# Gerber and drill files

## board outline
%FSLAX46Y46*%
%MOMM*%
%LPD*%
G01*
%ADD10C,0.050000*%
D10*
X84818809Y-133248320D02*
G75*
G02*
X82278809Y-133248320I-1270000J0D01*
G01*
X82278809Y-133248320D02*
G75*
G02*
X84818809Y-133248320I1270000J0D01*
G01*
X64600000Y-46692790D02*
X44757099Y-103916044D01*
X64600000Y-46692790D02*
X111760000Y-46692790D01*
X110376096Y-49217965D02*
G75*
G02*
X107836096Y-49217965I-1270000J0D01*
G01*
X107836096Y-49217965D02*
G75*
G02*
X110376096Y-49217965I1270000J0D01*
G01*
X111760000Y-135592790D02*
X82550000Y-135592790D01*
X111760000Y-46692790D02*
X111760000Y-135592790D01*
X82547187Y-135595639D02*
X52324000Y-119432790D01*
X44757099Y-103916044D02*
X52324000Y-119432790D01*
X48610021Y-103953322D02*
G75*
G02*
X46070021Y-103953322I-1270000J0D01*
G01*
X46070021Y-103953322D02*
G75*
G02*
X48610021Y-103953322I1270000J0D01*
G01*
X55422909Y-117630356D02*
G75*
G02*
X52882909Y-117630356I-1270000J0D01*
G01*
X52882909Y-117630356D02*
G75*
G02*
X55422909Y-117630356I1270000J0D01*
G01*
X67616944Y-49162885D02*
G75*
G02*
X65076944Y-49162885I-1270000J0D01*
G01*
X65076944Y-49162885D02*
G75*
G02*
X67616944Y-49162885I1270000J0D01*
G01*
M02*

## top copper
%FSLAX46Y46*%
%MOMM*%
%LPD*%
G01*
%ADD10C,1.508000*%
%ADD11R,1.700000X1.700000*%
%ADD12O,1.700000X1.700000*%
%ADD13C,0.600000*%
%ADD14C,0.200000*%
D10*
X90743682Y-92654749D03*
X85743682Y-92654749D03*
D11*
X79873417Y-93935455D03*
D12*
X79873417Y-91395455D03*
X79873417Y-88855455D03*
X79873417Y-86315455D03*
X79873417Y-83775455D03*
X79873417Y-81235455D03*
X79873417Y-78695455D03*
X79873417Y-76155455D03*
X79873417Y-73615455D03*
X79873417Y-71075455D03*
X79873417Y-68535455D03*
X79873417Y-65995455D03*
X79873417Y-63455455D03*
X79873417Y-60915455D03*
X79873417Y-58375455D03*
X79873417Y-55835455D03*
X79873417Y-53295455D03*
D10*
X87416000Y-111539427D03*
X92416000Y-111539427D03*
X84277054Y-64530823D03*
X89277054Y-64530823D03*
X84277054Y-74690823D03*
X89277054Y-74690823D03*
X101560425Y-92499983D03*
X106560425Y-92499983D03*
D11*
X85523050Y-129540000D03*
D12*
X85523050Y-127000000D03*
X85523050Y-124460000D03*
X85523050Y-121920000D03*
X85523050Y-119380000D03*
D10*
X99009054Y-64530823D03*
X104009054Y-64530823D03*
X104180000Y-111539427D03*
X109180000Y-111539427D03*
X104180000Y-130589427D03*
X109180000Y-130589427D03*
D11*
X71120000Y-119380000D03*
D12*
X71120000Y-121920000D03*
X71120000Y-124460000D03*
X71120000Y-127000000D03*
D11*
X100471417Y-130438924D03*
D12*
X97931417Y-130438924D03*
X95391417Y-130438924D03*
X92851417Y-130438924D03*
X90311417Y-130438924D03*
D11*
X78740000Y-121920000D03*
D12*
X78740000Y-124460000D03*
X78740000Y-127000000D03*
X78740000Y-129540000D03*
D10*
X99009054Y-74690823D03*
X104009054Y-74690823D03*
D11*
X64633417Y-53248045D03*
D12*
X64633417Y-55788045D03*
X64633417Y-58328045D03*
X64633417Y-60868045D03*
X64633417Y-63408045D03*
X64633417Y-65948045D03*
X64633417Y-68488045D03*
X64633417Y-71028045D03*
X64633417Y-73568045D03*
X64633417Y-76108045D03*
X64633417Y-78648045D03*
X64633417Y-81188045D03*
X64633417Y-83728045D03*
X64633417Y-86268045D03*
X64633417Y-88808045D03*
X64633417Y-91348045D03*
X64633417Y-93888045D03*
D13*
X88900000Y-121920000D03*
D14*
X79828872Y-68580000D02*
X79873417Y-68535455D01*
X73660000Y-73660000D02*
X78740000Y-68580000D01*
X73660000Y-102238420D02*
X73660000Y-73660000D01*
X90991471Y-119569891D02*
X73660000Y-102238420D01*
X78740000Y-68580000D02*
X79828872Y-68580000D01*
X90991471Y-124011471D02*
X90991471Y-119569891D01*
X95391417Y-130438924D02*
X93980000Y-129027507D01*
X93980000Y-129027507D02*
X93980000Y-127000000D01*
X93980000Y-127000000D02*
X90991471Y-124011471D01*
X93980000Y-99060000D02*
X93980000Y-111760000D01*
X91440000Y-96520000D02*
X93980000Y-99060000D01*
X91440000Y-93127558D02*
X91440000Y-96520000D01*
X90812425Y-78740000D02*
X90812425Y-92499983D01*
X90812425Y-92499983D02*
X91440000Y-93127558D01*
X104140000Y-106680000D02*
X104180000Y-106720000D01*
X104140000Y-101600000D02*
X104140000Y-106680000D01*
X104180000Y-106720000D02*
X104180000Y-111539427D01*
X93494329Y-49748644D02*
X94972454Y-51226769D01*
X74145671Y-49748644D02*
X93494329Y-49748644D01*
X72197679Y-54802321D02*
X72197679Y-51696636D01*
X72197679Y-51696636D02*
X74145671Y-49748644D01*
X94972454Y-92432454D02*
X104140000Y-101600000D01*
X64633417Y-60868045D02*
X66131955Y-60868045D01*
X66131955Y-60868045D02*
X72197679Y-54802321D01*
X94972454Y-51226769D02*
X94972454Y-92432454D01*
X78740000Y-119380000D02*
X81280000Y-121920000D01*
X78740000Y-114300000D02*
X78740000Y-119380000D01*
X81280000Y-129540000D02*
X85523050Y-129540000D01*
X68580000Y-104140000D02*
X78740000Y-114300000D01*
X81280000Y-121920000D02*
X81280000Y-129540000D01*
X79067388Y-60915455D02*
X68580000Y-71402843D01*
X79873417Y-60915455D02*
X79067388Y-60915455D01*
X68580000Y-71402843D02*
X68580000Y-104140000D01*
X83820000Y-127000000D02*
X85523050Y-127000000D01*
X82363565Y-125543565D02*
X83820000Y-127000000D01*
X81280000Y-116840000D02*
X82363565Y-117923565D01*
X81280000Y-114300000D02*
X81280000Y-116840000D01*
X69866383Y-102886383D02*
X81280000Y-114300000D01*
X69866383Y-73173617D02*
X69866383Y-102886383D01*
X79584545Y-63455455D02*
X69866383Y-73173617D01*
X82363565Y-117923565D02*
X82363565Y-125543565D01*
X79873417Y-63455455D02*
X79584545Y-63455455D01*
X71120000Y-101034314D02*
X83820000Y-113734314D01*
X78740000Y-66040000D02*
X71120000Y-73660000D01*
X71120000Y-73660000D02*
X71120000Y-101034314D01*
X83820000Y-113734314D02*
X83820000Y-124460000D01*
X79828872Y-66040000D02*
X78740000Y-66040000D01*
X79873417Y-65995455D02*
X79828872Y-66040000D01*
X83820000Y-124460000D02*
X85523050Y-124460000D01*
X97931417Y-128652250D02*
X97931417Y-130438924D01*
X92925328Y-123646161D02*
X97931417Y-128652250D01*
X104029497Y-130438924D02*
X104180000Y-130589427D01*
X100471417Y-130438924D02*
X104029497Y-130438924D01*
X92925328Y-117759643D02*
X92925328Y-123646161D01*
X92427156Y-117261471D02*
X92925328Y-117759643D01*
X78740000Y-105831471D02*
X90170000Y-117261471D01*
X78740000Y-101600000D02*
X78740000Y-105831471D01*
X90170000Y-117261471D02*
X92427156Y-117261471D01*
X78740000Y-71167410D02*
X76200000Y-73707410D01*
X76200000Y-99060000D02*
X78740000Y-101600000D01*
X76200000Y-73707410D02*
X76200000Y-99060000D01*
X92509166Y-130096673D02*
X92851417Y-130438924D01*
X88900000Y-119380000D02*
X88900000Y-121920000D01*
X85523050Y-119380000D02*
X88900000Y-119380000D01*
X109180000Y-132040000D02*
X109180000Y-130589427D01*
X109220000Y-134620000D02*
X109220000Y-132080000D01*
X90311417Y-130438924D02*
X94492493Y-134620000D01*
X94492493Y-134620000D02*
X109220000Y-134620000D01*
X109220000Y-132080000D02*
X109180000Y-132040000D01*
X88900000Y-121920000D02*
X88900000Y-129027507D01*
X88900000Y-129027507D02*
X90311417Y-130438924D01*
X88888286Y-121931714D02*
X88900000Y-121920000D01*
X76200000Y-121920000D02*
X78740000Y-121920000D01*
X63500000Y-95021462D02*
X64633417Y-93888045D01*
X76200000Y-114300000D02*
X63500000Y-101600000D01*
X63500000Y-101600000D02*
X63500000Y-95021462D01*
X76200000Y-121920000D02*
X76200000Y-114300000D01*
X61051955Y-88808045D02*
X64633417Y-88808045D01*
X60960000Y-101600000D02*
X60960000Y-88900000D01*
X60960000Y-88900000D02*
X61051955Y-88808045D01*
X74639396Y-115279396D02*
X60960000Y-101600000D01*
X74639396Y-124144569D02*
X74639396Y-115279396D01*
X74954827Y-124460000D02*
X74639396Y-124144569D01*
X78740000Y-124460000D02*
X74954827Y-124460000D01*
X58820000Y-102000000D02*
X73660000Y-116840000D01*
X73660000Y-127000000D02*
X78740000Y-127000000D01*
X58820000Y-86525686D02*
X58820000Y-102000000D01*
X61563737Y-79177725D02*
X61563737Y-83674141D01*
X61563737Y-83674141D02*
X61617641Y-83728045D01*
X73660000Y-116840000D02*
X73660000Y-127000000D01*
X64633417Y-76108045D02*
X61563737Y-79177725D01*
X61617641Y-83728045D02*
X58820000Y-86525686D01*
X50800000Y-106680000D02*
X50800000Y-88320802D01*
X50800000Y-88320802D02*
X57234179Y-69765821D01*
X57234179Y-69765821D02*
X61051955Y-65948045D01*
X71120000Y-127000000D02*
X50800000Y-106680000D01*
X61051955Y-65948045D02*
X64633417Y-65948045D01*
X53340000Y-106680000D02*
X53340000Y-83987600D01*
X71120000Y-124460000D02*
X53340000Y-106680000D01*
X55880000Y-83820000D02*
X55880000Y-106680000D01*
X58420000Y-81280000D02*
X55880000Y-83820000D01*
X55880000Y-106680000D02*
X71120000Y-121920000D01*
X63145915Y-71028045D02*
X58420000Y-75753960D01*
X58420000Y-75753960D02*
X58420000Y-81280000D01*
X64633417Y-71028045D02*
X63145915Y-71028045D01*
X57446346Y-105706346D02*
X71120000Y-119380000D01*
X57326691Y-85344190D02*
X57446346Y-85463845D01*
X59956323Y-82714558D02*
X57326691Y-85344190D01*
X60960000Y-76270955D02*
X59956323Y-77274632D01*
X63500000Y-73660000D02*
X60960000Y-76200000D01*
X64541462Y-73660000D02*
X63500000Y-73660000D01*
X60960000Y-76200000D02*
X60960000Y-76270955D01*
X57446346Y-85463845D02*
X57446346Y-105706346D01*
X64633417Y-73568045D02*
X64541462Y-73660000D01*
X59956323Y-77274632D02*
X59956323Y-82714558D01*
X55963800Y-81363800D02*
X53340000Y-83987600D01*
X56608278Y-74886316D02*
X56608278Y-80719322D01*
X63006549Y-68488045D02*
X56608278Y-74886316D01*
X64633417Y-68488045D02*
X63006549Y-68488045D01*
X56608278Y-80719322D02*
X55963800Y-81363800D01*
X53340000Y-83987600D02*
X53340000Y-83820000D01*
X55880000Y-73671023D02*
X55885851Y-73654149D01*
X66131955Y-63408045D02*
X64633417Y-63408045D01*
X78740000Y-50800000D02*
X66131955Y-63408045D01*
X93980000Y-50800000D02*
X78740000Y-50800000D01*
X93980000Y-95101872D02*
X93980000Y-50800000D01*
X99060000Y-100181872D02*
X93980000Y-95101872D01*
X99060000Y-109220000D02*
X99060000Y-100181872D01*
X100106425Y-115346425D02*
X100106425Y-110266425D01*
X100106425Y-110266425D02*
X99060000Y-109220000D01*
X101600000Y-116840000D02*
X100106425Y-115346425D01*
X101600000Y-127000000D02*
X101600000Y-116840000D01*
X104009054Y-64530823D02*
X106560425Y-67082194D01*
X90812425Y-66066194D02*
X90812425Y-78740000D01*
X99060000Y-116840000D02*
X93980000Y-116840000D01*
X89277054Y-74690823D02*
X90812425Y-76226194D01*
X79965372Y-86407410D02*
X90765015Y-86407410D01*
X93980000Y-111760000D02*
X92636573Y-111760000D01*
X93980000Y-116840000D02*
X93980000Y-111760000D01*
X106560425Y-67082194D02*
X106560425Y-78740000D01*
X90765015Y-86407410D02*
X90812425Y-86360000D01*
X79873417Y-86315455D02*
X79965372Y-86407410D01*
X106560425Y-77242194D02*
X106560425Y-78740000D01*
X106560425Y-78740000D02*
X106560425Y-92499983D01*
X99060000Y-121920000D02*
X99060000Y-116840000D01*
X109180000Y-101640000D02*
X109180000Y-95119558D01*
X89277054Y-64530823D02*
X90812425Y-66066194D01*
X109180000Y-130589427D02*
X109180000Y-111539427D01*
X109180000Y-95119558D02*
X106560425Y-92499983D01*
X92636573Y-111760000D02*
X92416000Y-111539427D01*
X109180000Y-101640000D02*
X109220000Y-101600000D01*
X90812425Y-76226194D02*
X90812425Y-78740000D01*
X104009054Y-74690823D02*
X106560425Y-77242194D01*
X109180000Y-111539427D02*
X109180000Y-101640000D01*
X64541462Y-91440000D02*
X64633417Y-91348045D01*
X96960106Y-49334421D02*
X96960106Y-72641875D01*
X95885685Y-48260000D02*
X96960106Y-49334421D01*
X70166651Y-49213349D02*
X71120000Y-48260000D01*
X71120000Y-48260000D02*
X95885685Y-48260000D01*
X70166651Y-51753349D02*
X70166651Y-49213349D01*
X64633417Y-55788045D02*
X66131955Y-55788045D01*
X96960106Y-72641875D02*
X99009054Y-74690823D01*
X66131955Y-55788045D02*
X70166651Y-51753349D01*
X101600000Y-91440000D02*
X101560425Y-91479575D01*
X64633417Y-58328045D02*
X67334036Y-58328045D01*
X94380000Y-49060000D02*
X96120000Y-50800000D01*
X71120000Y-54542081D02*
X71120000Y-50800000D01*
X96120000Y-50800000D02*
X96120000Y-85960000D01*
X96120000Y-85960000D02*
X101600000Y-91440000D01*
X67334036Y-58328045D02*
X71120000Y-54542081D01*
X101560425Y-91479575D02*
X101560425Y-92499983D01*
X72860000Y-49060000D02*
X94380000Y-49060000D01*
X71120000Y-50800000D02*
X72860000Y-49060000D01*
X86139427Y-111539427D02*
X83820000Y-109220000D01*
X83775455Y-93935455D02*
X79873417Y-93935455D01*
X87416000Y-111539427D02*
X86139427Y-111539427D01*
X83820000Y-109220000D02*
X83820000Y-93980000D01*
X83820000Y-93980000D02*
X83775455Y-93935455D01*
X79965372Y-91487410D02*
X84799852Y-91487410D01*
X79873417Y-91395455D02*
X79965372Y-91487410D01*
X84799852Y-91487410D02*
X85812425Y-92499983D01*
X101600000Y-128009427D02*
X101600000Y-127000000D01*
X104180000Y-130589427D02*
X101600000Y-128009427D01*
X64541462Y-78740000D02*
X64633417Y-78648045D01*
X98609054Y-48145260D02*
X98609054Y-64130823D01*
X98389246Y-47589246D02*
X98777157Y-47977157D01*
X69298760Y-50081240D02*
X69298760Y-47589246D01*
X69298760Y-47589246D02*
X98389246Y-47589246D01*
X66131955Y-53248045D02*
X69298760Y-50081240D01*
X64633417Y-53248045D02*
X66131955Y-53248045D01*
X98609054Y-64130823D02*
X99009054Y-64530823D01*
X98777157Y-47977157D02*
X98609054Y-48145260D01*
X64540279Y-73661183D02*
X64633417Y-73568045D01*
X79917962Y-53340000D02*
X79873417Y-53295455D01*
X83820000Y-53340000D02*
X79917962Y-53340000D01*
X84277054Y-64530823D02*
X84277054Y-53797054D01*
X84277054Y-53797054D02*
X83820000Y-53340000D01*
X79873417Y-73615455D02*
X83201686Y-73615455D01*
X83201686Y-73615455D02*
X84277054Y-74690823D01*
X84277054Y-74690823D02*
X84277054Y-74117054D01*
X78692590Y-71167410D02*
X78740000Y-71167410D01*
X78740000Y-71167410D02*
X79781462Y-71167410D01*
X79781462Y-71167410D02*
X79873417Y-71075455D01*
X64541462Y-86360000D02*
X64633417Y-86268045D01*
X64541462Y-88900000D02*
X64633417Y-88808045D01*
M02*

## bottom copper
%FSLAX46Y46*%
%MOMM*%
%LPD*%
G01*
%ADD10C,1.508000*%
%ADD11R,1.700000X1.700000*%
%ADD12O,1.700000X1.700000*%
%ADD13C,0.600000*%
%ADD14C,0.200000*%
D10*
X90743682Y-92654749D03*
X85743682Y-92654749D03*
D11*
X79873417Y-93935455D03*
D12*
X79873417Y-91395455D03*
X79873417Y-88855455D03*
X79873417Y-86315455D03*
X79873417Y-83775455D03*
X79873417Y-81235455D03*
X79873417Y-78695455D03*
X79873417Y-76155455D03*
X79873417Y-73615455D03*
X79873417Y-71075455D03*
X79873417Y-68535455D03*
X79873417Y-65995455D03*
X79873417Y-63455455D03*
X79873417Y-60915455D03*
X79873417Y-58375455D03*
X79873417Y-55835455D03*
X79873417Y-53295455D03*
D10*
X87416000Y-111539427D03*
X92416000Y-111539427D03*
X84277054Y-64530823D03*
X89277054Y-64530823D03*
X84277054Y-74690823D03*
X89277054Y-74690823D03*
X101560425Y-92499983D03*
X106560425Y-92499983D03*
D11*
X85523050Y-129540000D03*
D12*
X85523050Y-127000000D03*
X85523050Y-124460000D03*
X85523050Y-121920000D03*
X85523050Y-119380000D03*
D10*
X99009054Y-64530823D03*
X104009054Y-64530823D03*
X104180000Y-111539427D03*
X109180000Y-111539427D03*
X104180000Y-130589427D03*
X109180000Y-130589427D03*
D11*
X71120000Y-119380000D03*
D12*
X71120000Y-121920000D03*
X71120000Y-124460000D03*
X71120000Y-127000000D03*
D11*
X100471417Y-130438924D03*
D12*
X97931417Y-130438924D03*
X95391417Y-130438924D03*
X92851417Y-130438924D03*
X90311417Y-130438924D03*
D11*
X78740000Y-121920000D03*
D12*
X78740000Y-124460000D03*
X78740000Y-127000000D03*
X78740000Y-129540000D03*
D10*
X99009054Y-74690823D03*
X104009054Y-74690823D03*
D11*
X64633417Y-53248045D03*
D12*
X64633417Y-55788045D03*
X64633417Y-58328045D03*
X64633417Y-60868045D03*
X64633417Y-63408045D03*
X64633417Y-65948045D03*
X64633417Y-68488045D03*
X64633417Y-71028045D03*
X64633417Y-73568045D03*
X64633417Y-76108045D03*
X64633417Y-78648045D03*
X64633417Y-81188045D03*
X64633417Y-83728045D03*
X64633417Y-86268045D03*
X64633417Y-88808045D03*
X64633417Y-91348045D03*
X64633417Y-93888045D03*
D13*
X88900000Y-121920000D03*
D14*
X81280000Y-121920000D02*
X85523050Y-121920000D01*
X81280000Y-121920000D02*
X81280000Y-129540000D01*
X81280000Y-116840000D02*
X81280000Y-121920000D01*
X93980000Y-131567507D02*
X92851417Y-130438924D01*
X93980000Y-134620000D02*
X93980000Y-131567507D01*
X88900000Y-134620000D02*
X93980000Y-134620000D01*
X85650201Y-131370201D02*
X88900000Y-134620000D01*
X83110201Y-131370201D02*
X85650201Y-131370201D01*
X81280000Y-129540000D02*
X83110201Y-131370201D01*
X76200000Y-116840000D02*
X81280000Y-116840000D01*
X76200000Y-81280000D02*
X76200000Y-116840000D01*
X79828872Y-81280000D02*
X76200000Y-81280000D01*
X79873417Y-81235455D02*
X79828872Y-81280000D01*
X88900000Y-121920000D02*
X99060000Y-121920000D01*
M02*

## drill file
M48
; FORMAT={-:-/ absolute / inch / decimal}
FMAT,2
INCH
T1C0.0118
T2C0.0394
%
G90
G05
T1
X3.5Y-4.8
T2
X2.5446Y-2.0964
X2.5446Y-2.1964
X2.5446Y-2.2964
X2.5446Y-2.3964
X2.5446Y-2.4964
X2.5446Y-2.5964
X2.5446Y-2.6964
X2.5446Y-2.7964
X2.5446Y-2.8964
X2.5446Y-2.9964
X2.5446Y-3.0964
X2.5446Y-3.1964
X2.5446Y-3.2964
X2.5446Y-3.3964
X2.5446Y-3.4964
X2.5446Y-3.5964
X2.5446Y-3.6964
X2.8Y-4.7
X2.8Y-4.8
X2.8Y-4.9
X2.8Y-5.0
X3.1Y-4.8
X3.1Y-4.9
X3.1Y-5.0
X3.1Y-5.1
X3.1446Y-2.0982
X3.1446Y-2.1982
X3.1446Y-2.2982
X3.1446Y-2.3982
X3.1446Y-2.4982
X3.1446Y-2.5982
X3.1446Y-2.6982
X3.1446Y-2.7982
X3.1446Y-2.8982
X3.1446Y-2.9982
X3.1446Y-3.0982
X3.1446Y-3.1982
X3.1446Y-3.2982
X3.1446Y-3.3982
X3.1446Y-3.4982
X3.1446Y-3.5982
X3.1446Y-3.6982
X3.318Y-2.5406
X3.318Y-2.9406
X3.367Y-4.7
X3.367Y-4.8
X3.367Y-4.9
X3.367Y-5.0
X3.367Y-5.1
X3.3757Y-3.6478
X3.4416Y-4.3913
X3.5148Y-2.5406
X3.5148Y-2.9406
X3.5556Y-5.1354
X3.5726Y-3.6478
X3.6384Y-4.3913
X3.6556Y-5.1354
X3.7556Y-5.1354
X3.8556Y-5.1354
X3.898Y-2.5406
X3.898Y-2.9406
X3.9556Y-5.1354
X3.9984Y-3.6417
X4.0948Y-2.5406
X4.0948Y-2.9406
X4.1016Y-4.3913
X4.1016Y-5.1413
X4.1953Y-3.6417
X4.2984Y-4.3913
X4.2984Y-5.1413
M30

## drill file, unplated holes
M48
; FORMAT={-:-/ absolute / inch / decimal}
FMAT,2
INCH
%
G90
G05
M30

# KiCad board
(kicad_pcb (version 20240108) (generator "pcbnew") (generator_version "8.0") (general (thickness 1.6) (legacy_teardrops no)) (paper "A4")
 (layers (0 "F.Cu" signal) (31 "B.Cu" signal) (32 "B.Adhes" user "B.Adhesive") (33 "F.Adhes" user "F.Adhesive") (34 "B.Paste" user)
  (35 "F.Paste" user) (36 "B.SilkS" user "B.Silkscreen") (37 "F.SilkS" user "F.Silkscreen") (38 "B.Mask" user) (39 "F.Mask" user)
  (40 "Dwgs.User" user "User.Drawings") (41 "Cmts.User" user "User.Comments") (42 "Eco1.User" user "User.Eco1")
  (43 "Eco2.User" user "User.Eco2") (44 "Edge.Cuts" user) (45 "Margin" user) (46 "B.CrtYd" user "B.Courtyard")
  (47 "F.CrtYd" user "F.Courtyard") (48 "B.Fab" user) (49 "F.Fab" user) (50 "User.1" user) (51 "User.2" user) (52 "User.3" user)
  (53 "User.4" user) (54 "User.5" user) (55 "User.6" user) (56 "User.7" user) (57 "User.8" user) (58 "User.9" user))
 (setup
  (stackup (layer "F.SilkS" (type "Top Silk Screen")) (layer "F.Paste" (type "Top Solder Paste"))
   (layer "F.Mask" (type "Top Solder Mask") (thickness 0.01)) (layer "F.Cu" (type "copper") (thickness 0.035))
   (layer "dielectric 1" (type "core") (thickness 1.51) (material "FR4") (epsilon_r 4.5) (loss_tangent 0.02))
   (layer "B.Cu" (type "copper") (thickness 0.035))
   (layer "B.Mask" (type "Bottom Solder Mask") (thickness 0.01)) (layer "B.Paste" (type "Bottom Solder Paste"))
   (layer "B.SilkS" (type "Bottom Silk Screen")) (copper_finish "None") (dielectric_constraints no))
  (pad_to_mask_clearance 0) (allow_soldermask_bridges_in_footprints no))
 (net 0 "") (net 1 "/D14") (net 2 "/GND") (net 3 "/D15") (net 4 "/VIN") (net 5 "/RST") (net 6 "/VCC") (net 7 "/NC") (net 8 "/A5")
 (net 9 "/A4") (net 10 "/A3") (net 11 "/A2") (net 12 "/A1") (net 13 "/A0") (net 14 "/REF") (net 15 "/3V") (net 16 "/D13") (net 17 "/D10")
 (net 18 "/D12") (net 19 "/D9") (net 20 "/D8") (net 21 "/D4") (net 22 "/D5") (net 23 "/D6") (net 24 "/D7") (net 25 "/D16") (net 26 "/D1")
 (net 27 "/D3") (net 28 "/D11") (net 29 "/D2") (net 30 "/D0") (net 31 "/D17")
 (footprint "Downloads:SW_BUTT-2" (layer "F.Cu") (at 88.243682 92.654749)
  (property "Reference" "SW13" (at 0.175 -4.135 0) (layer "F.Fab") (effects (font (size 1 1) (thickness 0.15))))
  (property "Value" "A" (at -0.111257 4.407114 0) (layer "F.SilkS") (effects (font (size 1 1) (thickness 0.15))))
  (pad "1" thru_hole circle (at -2.5 0) (size 1.508 1.508) (drill 1) (layers "*.Cu" "*.Mask") (remove_unused_layers no) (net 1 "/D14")
   (solder_mask_margin 0.102))
  (pad "2" thru_hole circle (at 2.5 0) (size 1.508 1.508) (drill 1) (layers "*.Cu" "*.Mask") (remove_unused_layers no) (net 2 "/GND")
   (solder_mask_margin 0.102)))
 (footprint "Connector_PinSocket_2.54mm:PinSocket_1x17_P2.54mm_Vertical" (layer "F.Cu") (at 79.873417 93.935455 180)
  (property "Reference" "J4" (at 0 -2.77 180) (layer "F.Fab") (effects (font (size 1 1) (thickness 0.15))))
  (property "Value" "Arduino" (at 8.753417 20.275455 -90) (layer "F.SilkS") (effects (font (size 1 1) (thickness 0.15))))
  (pad "1" thru_hole rect (at 0 0 180) (size 1.7 1.7) (drill 1) (layers "*.Cu" "*.Mask") (remove_unused_layers no) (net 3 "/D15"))
  (pad "2" thru_hole oval (at 0 2.54 180) (size 1.7 1.7) (drill 1) (layers "*.Cu" "*.Mask") (remove_unused_layers no) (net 1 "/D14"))
  (pad "3" thru_hole oval (at 0 5.08 180) (size 1.7 1.7) (drill 1) (layers "*.Cu" "*.Mask") (remove_unused_layers no) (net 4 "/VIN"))
  (pad "4" thru_hole oval (at 0 7.62 180) (size 1.7 1.7) (drill 1) (layers "*.Cu" "*.Mask") (remove_unused_layers no) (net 2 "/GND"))
  (pad "5" thru_hole oval (at 0 10.16 180) (size 1.7 1.7) (drill 1) (layers "*.Cu" "*.Mask") (remove_unused_layers no) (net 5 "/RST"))
  (pad "6" thru_hole oval (at 0 12.7 180) (size 1.7 1.7) (drill 1) (layers "*.Cu" "*.Mask") (remove_unused_layers no) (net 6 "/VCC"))
  (pad "7" thru_hole oval (at 0 15.24 180) (size 1.7 1.7) (drill 1) (layers "*.Cu" "*.Mask") (remove_unused_layers no) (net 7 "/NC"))
  (pad "8" thru_hole oval (at 0 17.78 180) (size 1.7 1.7) (drill 1) (layers "*.Cu" "*.Mask") (remove_unused_layers no) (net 7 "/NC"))
  (pad "9" thru_hole oval (at 0 20.32 180) (size 1.7 1.7) (drill 1) (layers "*.Cu" "*.Mask") (remove_unused_layers no) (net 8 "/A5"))
  (pad "10" thru_hole oval (at 0 22.86 180) (size 1.7 1.7) (drill 1) (layers "*.Cu" "*.Mask") (remove_unused_layers no) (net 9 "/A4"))
  (pad "11" thru_hole oval (at 0 25.4 180) (size 1.7 1.7) (drill 1) (layers "*.Cu" "*.Mask") (remove_unused_layers no) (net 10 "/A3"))
  (pad "12" thru_hole oval (at 0 27.94 180) (size 1.7 1.7) (drill 1) (layers "*.Cu" "*.Mask") (remove_unused_layers no) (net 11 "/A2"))
  (pad "13" thru_hole oval (at 0 30.48 180) (size 1.7 1.7) (drill 1) (layers "*.Cu" "*.Mask") (remove_unused_layers no) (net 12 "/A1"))
  (pad "14" thru_hole oval (at 0 33.02 180) (size 1.7 1.7) (drill 1) (layers "*.Cu" "*.Mask") (remove_unused_layers no) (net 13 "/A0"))
  (pad "15" thru_hole oval (at 0 35.56 180) (size 1.7 1.7) (drill 1) (layers "*.Cu" "*.Mask") (remove_unused_layers no) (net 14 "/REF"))
  (pad "16" thru_hole oval (at 0 38.1 180) (size 1.7 1.7) (drill 1) (layers "*.Cu" "*.Mask") (remove_unused_layers no) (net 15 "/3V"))
  (pad "17" thru_hole oval (at 0 40.64 180) (size 1.7 1.7) (drill 1) (layers "*.Cu" "*.Mask") (remove_unused_layers no) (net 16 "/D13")))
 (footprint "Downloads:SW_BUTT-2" (layer "F.Cu") (at 89.916 111.539427)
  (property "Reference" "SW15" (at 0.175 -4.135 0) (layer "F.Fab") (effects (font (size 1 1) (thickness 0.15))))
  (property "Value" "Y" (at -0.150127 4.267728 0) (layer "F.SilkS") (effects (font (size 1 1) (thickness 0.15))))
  (pad "1" thru_hole circle (at -2.5 0) (size 1.508 1.508) (drill 1) (layers "*.Cu" "*.Mask") (remove_unused_layers no) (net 3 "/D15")
   (solder_mask_margin 0.102))
  (pad "2" thru_hole circle (at 2.5 0) (size 1.508 1.508) (drill 1) (layers "*.Cu" "*.Mask") (remove_unused_layers no) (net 2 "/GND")
   (solder_mask_margin 0.102)))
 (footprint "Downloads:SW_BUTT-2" (layer "F.Cu") (at 86.777054 64.530823)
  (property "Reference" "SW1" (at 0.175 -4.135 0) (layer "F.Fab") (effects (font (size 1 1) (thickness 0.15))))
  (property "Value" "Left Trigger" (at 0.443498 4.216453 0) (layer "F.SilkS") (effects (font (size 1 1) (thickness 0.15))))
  (pad "1" thru_hole circle (at -2.5 0) (size 1.508 1.508) (drill 1) (layers "*.Cu" "*.Mask") (remove_unused_layers no) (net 16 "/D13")
   (solder_mask_margin 0.102))
  (pad "2" thru_hole circle (at 2.5 0) (size 1.508 1.508) (drill 1) (layers "*.Cu" "*.Mask") (remove_unused_layers no) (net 2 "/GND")
   (solder_mask_margin 0.102)))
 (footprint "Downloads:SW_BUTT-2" (layer "F.Cu") (at 86.777054 74.690823)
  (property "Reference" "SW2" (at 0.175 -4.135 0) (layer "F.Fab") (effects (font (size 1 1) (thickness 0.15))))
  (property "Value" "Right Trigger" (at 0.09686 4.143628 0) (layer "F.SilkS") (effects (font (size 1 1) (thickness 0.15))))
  (pad "1" thru_hole circle (at -2.5 0) (size 1.508 1.508) (drill 1) (layers "*.Cu" "*.Mask") (remove_unused_layers no) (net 8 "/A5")
   (solder_mask_margin 0.102))
  (pad "2" thru_hole circle (at 2.5 0) (size 1.508 1.508) (drill 1) (layers "*.Cu" "*.Mask") (remove_unused_layers no) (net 2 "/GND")
   (solder_mask_margin 0.102)))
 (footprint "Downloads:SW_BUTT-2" (layer "F.Cu") (at 104.060425 92.499983)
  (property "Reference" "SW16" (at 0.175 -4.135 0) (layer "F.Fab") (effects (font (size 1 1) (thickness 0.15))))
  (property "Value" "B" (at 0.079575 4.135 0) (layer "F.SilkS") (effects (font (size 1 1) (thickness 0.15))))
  (pad "1" thru_hole circle (at -2.5 0) (size 1.508 1.508) (drill 1) (layers "*.Cu" "*.Mask") (remove_unused_layers no) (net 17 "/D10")
   (solder_mask_margin 0.102))
  (pad "2" thru_hole circle (at 2.5 0) (size 1.508 1.508) (drill 1) (layers "*.Cu" "*.Mask") (remove_unused_layers no) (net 2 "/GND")
   (solder_mask_margin 0.102)))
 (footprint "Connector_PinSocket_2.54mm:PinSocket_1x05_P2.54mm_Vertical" (layer "F.Cu") (at 85.52305 129.54 180)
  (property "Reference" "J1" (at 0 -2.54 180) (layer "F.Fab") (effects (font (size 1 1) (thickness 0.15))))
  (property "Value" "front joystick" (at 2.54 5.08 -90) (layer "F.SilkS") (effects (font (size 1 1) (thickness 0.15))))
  (pad "1" thru_hole rect (at 0 0 180) (size 1.7 1.7) (drill 1) (layers "*.Cu" "*.Mask") (remove_unused_layers no) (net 13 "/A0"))
  (pad "2" thru_hole oval (at 0 2.54 180) (size 1.7 1.7) (drill 1) (layers "*.Cu" "*.Mask") (remove_unused_layers no) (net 12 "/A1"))
  (pad "3" thru_hole oval (at 0 5.08 180) (size 1.7 1.7) (drill 1) (layers "*.Cu" "*.Mask") (remove_unused_layers no) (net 11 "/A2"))
  (pad "4" thru_hole oval (at 0 7.62 180) (size 1.7 1.7) (drill 1) (layers "*.Cu" "*.Mask") (remove_unused_layers no) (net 6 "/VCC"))
  (pad "5" thru_hole oval (at 0 10.16 180) (size 1.7 1.7) (drill 1) (layers "*.Cu" "*.Mask") (remove_unused_layers no) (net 2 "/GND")))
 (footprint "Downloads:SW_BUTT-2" (layer "F.Cu") (at 101.509054 64.530823)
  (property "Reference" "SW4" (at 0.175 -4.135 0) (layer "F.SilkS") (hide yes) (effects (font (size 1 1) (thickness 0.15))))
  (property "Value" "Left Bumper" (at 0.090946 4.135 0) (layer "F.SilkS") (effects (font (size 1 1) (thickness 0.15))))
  (pad "1" thru_hole circle (at -2.5 0) (size 1.508 1.508) (drill 1) (layers "*.Cu" "*.Mask") (remove_unused_layers no) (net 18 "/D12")
   (solder_mask_margin 0.102))
  (pad "2" thru_hole circle (at 2.5 0) (size 1.508 1.508) (drill 1) (layers "*.Cu" "*.Mask") (remove_unused_layers no) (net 2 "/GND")
   (solder_mask_margin 0.102)))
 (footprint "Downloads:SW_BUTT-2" (layer "F.Cu") (at 106.68 111.539427)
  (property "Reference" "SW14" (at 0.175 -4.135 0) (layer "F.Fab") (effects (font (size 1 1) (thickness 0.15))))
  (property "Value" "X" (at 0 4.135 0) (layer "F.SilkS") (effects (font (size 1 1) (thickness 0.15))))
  (pad "1" thru_hole circle (at -2.5 0) (size 1.508 1.508) (drill 1) (layers "*.Cu" "*.Mask") (remove_unused_layers no) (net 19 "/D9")
   (solder_mask_margin 0.102))
  (pad "2" thru_hole circle (at 2.5 0) (size 1.508 1.508) (drill 1) (layers "*.Cu" "*.Mask") (remove_unused_layers no) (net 2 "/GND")
   (solder_mask_margin 0.102)))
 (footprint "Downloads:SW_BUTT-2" (layer "F.Cu") (at 106.68 130.589427)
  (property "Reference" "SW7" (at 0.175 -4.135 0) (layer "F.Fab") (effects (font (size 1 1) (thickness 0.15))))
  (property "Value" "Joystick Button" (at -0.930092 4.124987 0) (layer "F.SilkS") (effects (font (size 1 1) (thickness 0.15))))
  (pad "1" thru_hole circle (at -2.5 0) (size 1.508 1.508) (drill 1) (layers "*.Cu" "*.Mask") (remove_unused_layers no) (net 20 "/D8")
   (solder_mask_margin 0.102))
  (pad "2" thru_hole circle (at 2.5 0) (size 1.508 1.508) (drill 1) (layers "*.Cu" "*.Mask") (remove_unused_layers no) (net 2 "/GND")
   (solder_mask_margin 0.102)))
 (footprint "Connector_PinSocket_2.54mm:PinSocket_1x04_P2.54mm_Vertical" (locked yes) (layer "F.Cu") (at 71.12 119.38)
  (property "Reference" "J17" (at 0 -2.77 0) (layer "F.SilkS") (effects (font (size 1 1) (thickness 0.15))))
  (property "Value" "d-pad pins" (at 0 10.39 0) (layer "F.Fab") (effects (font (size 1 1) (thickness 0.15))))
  (pad "1" thru_hole rect (at 0 0) (size 1.7 1.7) (drill 1) (layers "*.Cu" "*.Mask") (remove_unused_layers no) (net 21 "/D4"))
  (pad "2" thru_hole oval (at 0 2.54) (size 1.7 1.7) (drill 1) (layers "*.Cu" "*.Mask") (remove_unused_layers no) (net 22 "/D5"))
  (pad "3" thru_hole oval (at 0 5.08) (size 1.7 1.7) (drill 1) (layers "*.Cu" "*.Mask") (remove_unused_layers no) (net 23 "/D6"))
  (pad "4" thru_hole oval (at 0 7.62) (size 1.7 1.7) (drill 1) (layers "*.Cu" "*.Mask") (remove_unused_layers no) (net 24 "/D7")))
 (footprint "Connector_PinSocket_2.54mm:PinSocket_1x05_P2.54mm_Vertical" (layer "F.Cu") (at 100.471417 130.438924 -90)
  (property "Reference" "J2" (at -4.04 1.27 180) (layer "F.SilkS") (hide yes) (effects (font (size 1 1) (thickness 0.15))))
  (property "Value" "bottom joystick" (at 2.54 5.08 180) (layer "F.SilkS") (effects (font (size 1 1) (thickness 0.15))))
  (pad "1" thru_hole rect (at 0 0 270) (size 1.7 1.7) (drill 1) (layers "*.Cu" "*.Mask") (remove_unused_layers no) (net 20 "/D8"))
  (pad "2" thru_hole oval (at 0 2.54 270) (size 1.7 1.7) (drill 1) (layers "*.Cu" "*.Mask") (remove_unused_layers no) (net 9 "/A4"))
  (pad "3" thru_hole oval (at 0 5.08 270) (size 1.7 1.7) (drill 1) (layers "*.Cu" "*.Mask") (remove_unused_layers no) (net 10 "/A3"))
  (pad "4" thru_hole oval (at 0 7.62 270) (size 1.7 1.7) (drill 1) (layers "*.Cu" "*.Mask") (remove_unused_layers no) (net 6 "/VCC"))
  (pad "5" thru_hole oval (at 0 10.16 270) (size 1.7 1.7) (drill 1) (layers "*.Cu" "*.Mask") (remove_unused_layers no) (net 2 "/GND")))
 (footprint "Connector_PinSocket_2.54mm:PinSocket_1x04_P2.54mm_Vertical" (layer "F.Cu") (at 78.74 121.92)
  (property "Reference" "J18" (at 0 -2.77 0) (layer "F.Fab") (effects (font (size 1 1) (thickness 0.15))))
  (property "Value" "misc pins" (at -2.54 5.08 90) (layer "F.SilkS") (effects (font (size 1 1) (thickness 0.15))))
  (pad "1" thru_hole rect (at 0 0) (size 1.7 1.7) (drill 1) (layers "*.Cu" "*.Mask") (remove_unused_layers no) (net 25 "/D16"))
  (pad "2" thru_hole oval (at 0 2.54) (size 1.7 1.7) (drill 1) (layers "*.Cu" "*.Mask") (remove_unused_layers no) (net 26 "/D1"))
  (pad "3" thru_hole oval (at 0 5.08) (size 1.7 1.7) (drill 1) (layers "*.Cu" "*.Mask") (remove_unused_layers no) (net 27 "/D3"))
  (pad "4" thru_hole oval (at 0 7.62) (size 1.7 1.7) (drill 1) (layers "*.Cu" "*.Mask") (remove_unused_layers no) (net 2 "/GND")))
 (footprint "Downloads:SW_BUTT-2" (layer "F.Cu") (at 101.509054 74.690823)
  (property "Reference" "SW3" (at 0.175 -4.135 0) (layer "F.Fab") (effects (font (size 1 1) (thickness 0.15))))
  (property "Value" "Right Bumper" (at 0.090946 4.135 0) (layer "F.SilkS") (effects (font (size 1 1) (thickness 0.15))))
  (pad "1" thru_hole circle (at -2.5 0) (size 1.508 1.508) (drill 1) (layers "*.Cu" "*.Mask") (remove_unused_layers no) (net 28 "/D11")
   (solder_mask_margin 0.102))
  (pad "2" thru_hole circle (at 2.5 0) (size 1.508 1.508) (drill 1) (layers "*.Cu" "*.Mask") (remove_unused_layers no) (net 2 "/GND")
   (solder_mask_margin 0.102)))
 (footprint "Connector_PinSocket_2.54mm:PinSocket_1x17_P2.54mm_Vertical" (layer "F.Cu") (at 64.633417 53.248045)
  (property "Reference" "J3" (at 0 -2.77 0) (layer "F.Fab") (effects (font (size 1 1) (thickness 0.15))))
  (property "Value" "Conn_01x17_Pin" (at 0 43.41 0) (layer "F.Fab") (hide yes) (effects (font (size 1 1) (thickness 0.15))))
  (pad "1" thru_hole rect (at 0 0) (size 1.7 1.7) (drill 1) (layers "*.Cu" "*.Mask") (remove_unused_layers no) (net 18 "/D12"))
  (pad "2" thru_hole oval (at 0 2.54) (size 1.7 1.7) (drill 1) (layers "*.Cu" "*.Mask") (remove_unused_layers no) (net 28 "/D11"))
  (pad "3" thru_hole oval (at 0 5.08) (size 1.7 1.7) (drill 1) (layers "*.Cu" "*.Mask") (remove_unused_layers no) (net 17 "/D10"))
  (pad "4" thru_hole oval (at 0 7.62) (size 1.7 1.7) (drill 1) (layers "*.Cu" "*.Mask") (remove_unused_layers no) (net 19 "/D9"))
  (pad "5" thru_hole oval (at 0 10.16) (size 1.7 1.7) (drill 1) (layers "*.Cu" "*.Mask") (remove_unused_layers no) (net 20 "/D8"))
  (pad "6" thru_hole oval (at 0 12.7) (size 1.7 1.7) (drill 1) (layers "*.Cu" "*.Mask") (remove_unused_layers no) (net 24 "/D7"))
  (pad "7" thru_hole oval (at 0 15.24) (size 1.7 1.7) (drill 1) (layers "*.Cu" "*.Mask") (remove_unused_layers no) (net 23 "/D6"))
  (pad "8" thru_hole oval (at 0 17.78) (size 1.7 1.7) (drill 1) (layers "*.Cu" "*.Mask") (remove_unused_layers no) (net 22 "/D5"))
  (pad "9" thru_hole oval (at 0 20.32) (size 1.7 1.7) (drill 1) (layers "*.Cu" "*.Mask") (remove_unused_layers no) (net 21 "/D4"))
  (pad "10" thru_hole oval (at 0 22.86) (size 1.7 1.7) (drill 1) (layers "*.Cu" "*.Mask") (remove_unused_layers no) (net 27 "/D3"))
  (pad "11" thru_hole oval (at 0 25.4) (size 1.7 1.7) (drill 1) (layers "*.Cu" "*.Mask") (remove_unused_layers no) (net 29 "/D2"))
  (pad "12" thru_hole oval (at 0 27.94) (size 1.7 1.7) (drill 1) (layers "*.Cu" "*.Mask") (remove_unused_layers no) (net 2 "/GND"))
  (pad "13" thru_hole oval (at 0 30.48) (size 1.7 1.7) (drill 1) (layers "*.Cu" "*.Mask") (remove_unused_layers no) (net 5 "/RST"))
  (pad "14" thru_hole oval (at 0 33.02) (size 1.7 1.7) (drill 1) (layers "*.Cu" "*.Mask") (remove_unused_layers no) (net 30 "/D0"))
  (pad "15" thru_hole oval (at 0 35.56) (size 1.7 1.7) (drill 1) (layers "*.Cu" "*.Mask") (remove_unused_layers no) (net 26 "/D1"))
  (pad "16" thru_hole oval (at 0 38.1) (size 1.7 1.7) (drill 1) (layers "*.Cu" "*.Mask") (remove_unused_layers no) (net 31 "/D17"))
  (pad "17" thru_hole oval (at 0 40.64) (size 1.7 1.7) (drill 1) (layers "*.Cu" "*.Mask") (remove_unused_layers no) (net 25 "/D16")))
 (gr_line (start 64.6 46.69279) (end 44.757099 103.916044) (stroke (width 0.05) (type default)) (layer "Edge.Cuts"))
 (gr_line (start 64.6 46.69279) (end 111.76 46.69279) (stroke (width 0.05) (type default)) (layer "Edge.Cuts"))
 (gr_circle (center 83.548809 133.24832) (end 82.278809 133.24832) (stroke (width 0.05) (type default)) (fill none) (layer "Edge.Cuts"))
 (gr_circle (center 109.106096 49.217965) (end 110.376096 49.217965) (stroke (width 0.05) (type default)) (fill none) (layer "Edge.Cuts"))
 (gr_line (start 111.76 135.59279) (end 82.55 135.59279) (stroke (width 0.05) (type default)) (layer "Edge.Cuts"))
 (gr_line (start 111.76 46.69279) (end 111.76 135.59279) (stroke (width 0.05) (type default)) (layer "Edge.Cuts"))
 (gr_line (start 82.547187 135.595639) (end 52.324 119.43279) (stroke (width 0.05) (type default)) (layer "Edge.Cuts"))
 (gr_line (start 44.757099 103.916044) (end 52.324 119.43279) (stroke (width 0.05) (type default)) (layer "Edge.Cuts"))
 (gr_circle (center 47.340021 103.953322) (end 46.070021 103.953322) (stroke (width 0.05) (type default)) (fill none) (layer "Edge.Cuts"))
 (gr_circle (center 54.152909 117.630356) (end 52.882909 117.630356) (stroke (width 0.05) (type default)) (fill none) (layer "Edge.Cuts"))
 (gr_circle (center 66.346944 49.162885) (end 66.346944 47.892885) (stroke (width 0.05) (type default)) (fill none) (layer "Edge.Cuts"))
 (segment (start 66.131955 63.408045) (end 64.633417 63.408045) (width 0.2) (layer "F.Cu") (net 20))
 (segment (start 93.98 50.8) (end 78.74 50.8) (width 0.2) (layer "F.Cu") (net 20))
 (segment (start 100.471417 130.438924) (end 104.029497 130.438924) (width 0.2) (layer "F.Cu") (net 20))
 (segment (start 101.6 127) (end 101.6 116.84) (width 0.2) (layer "F.Cu") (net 20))
 (segment (start 100.106425 110.266425) (end 99.06 109.22) (width 0.2) (layer "F.Cu") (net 20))
 (segment (start 99.06 100.181872) (end 93.98 95.101872) (width 0.2) (layer "F.Cu") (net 20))
 (segment (start 100.106425 115.346425) (end 100.106425 110.266425) (width 0.2) (layer "F.Cu") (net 20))
 (segment (start 104.029497 130.438924) (end 104.18 130.589427) (width 0.2) (layer "F.Cu") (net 20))
 (segment (start 99.06 109.22) (end 99.06 100.181872) (width 0.2) (layer "F.Cu") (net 20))
 (segment (start 101.6 128.009427) (end 101.6 127) (width 0.2) (layer "F.Cu") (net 20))
 (segment (start 101.6 116.84) (end 100.106425 115.346425) (width 0.2) (layer "F.Cu") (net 20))
 (segment (start 78.74 50.8) (end 66.131955 63.408045) (width 0.2) (layer "F.Cu") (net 20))
 (segment (start 93.98 95.101872) (end 93.98 50.8) (width 0.2) (layer "F.Cu") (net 20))
 (segment (start 104.18 130.589427) (end 101.6 128.009427) (width 0.2) (layer "F.Cu") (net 20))
 (segment (start 92.509166 130.096673) (end 92.851417 130.438924) (width 0.2) (layer "F.Cu") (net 6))
 (segment (start 83.110201 131.370201) (end 85.650201 131.370201) (width 0.2) (layer "B.Cu") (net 6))
 (segment (start 81.28 121.92) (end 85.52305 121.92) (width 0.2) (layer "B.Cu") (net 6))
 (segment (start 81.28 116.84) (end 81.28 121.92) (width 0.2) (layer "B.Cu") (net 6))
 (segment (start 76.2 116.84) (end 81.28 116.84) (width 0.2) (layer "B.Cu") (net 6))
 (segment (start 88.9 134.62) (end 93.98 134.62) (width 0.2) (layer "B.Cu") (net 6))
 (segment (start 79.873417 81.235455) (end 79.828872 81.28) (width 0.2) (layer "B.Cu") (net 6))
 (segment (start 79.828872 81.28) (end 76.2 81.28) (width 0.2) (layer "B.Cu") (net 6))
 (segment (start 85.650201 131.370201) (end 88.9 134.62) (width 0.2) (layer "B.Cu") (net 6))
 (segment (start 81.28 129.54) (end 83.110201 131.370201) (width 0.2) (layer "B.Cu") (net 6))
 (segment (start 76.2 81.28) (end 76.2 116.84) (width 0.2) (layer "B.Cu") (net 6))
 (segment (start 93.98 134.62) (end 93.98 131.567507) (width 0.2) (layer "B.Cu") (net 6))
 (segment (start 93.98 131.567507) (end 92.851417 130.438924) (width 0.2) (layer "B.Cu") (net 6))
 (segment (start 81.28 121.92) (end 81.28 129.54) (width 0.2) (layer "B.Cu") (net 6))
 (segment (start 68.58 104.14) (end 78.74 114.3) (width 0.2) (layer "F.Cu") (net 13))
 (segment (start 79.067388 60.915455) (end 68.58 71.402843) (width 0.2) (layer "F.Cu") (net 13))
 (segment (start 81.28 129.54) (end 85.52305 129.54) (width 0.2) (layer "F.Cu") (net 13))
 (segment (start 79.873417 60.915455) (end 79.067388 60.915455) (width 0.2) (layer "F.Cu") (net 13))
 (segment (start 81.28 121.92) (end 81.28 129.54) (width 0.2) (layer "F.Cu") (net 13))
 (segment (start 78.74 114.3) (end 78.74 119.38) (width 0.2) (layer "F.Cu") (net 13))
 (segment (start 78.74 119.38) (end 81.28 121.92) (width 0.2) (layer "F.Cu") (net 13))
 (segment (start 68.58 71.402843) (end 68.58 104.14) (width 0.2) (layer "F.Cu") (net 13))
 (segment (start 104.009054 64.530823) (end 106.560425 67.082194) (width 0.2) (layer "F.Cu") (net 2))
 (segment (start 90.812425 66.066194) (end 90.812425 78.74) (width 0.2) (layer "F.Cu") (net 2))
 (segment (start 90.812425 78.74) (end 90.812425 92.499983) (width 0.2) (layer "F.Cu") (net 2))
 (segment (start 91.44 93.127558) (end 91.44 96.52) (width 0.2) (layer "F.Cu") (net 2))
 (segment (start 99.06 116.84) (end 93.98 116.84) (width 0.2) (layer "F.Cu") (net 2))
 (segment (start 89.277054 74.690823) (end 90.812425 76.226194) (width 0.2) (layer "F.Cu") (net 2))
 (segment (start 79.965372 86.40741) (end 90.765015 86.40741) (width 0.2) (layer "F.Cu") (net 2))
 (segment (start 88.9 121.92) (end 88.9 129.027507) (width 0.2) (layer "F.Cu") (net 2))
 (segment (start 93.98 111.76) (end 92.636573 111.76) (width 0.2) (layer "F.Cu") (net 2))
 (segment (start 93.98 116.84) (end 93.98 111.76) (width 0.2) (layer "F.Cu") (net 2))
 (segment (start 106.560425 67.082194) (end 106.560425 78.74) (width 0.2) (layer "F.Cu") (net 2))
 (segment (start 85.52305 119.38) (end 88.9 119.38) (width 0.2) (layer "F.Cu") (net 2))
 (segment (start 88.9 129.027507) (end 90.311417 130.438924) (width 0.2) (layer "F.Cu") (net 2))
 (segment (start 91.44 96.52) (end 93.98 99.06) (width 0.2) (layer "F.Cu") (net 2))
 (segment (start 90.765015 86.40741) (end 90.812425 86.36) (width 0.2) (layer "F.Cu") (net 2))
 (segment (start 88.9 119.38) (end 88.9 121.92) (width 0.2) (layer "F.Cu") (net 2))
 (segment (start 79.873417 86.315455) (end 79.965372 86.40741) (width 0.2) (layer "F.Cu") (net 2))
 (segment (start 106.560425 77.242194) (end 106.560425 78.74) (width 0.2) (layer "F.Cu") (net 2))
 (segment (start 106.560425 78.74) (end 106.560425 92.499983) (width 0.2) (layer "F.Cu") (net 2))
 (segment (start 109.22 132.08) (end 109.18 132.04) (width 0.2) (layer "F.Cu") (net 2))
 (segment (start 99.06 121.92) (end 99.06 116.84) (width 0.2) (layer "F.Cu") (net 2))
 (segment (start 109.18 101.64) (end 109.18 95.119558) (width 0.2) (layer "F.Cu") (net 2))
 (segment (start 89.277054 64.530823) (end 90.812425 66.066194) (width 0.2) (layer "F.Cu") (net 2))
 (segment (start 90.311417 130.438924) (end 94.492493 134.62) (width 0.2) (layer "F.Cu") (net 2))
 (segment (start 88.888286 121.931714) (end 88.9 121.92) (width 0.2) (layer "F.Cu") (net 2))
 (segment (start 109.18 130.589427) (end 109.18 111.539427) (width 0.2) (layer "F.Cu") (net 2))
 (segment (start 90.812425 92.499983) (end 91.44 93.127558) (width 0.2) (layer "F.Cu") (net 2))
 (segment (start 109.18 95.119558) (end 106.560425 92.499983) (width 0.2) (layer "F.Cu") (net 2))
 (segment (start 92.636573 111.76) (end 92.416 111.539427) (width 0.2) (layer "F.Cu") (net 2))
 (segment (start 94.492493 134.62) (end 109.22 134.62) (width 0.2) (layer "F.Cu") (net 2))
 (segment (start 109.22 134.62) (end 109.22 132.08) (width 0.2) (layer "F.Cu") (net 2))
 (segment (start 109.18 101.64) (end 109.22 101.6) (width 0.2) (layer "F.Cu") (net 2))
 (segment (start 90.812425 76.226194) (end 90.812425 78.74) (width 0.2) (layer "F.Cu") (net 2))
 (segment (start 104.009054 74.690823) (end 106.560425 77.242194) (width 0.2) (layer "F.Cu") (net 2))
 (segment (start 109.18 111.539427) (end 109.18 101.64) (width 0.2) (layer "F.Cu") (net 2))
 (segment (start 93.98 99.06) (end 93.98 111.76) (width 0.2) (layer "F.Cu") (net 2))
 (segment (start 109.18 132.04) (end 109.18 130.589427) (width 0.2) (layer "F.Cu") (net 2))
 (via (at 88.9 121.92) (size 0.6) (drill 0.3) (layers "F.Cu" "B.Cu") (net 2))
 (segment (start 88.9 121.92) (end 99.06 121.92) (width 0.2) (layer "B.Cu") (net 2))
 (segment (start 69.866383 73.173617) (end 69.866383 102.886383) (width 0.2) (layer "F.Cu") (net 12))
 (segment (start 82.363565 117.923565) (end 82.363565 125.543565) (width 0.2) (layer "F.Cu") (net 12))
 (segment (start 81.28 114.3) (end 81.28 116.84) (width 0.2) (layer "F.Cu") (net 12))
 (segment (start 79.873417 63.455455) (end 79.584545 63.455455) (width 0.2) (layer "F.Cu") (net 12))
 (segment (start 79.584545 63.455455) (end 69.866383 73.173617) (width 0.2) (layer "F.Cu") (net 12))
 (segment (start 82.363565 125.543565) (end 83.82 127) (width 0.2) (layer "F.Cu") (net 12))
 (segment (start 81.28 116.84) (end 82.363565 117.923565) (width 0.2) (layer "F.Cu") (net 12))
 (segment (start 69.866383 102.886383) (end 81.28 114.3) (width 0.2) (layer "F.Cu") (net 12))
 (segment (start 83.82 127) (end 85.52305 127) (width 0.2) (layer "F.Cu") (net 12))
 (segment (start 76.2 121.92) (end 78.74 121.92) (width 0.2) (layer "F.Cu") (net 25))
 (segment (start 63.5 95.021462) (end 64.633417 93.888045) (width 0.2) (layer "F.Cu") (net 25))
 (segment (start 63.5 101.6) (end 63.5 95.021462) (width 0.2) (layer "F.Cu") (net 25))
 (segment (start 76.2 114.3) (end 63.5 101.6) (width 0.2) (layer "F.Cu") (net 25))
 (segment (start 76.2 121.92) (end 76.2 114.3) (width 0.2) (layer "F.Cu") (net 25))
 (segment (start 56.608278 80.719322) (end 55.9638 81.3638) (width 0.2) (layer "F.Cu") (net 23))
 (segment (start 56.608278 74.886316) (end 56.608278 80.719322) (width 0.2) (layer "F.Cu") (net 23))
 (segment (start 64.633417 68.488045) (end 63.006549 68.488045) (width 0.2) (layer "F.Cu") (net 23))
 (segment (start 71.12 124.46) (end 53.34 106.68) (width 0.2) (layer "F.Cu") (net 23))
 (segment (start 53.34 83.9876) (end 53.34 83.82) (width 0.2) (layer "F.Cu") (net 23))
 (segment (start 55.9638 81.3638) (end 53.34 83.9876) (width 0.2) (layer "F.Cu") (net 23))
 (segment (start 63.006549 68.488045) (end 56.608278 74.886316) (width 0.2) (layer "F.Cu") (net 23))
 (segment (start 53.34 106.68) (end 53.34 83.9876) (width 0.2) (layer "F.Cu") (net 23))
 (segment (start 55.88 73.671023) (end 55.885851 73.654149) (width 0.2) (layer "F.Cu") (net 24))
 (segment (start 50.8 88.320802) (end 57.234179 69.765821) (width 0.2) (layer "F.Cu") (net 24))
 (segment (start 61.051955 65.948045) (end 64.633417 65.948045) (width 0.2) (layer "F.Cu") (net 24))
 (segment (start 50.8 106.68) (end 50.8 88.320802) (width 0.2) (layer "F.Cu") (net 24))
 (segment (start 71.12 127) (end 50.8 106.68) (width 0.2) (layer "F.Cu") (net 24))
 (segment (start 57.234179 69.765821) (end 61.051955 65.948045) (width 0.2) (layer "F.Cu") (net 24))
 (segment (start 64.541462 91.44) (end 64.633417 91.348045) (width 0.2) (layer "F.Cu") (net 31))
 (segment (start 96.960106 49.334421) (end 96.960106 72.641875) (width 0.2) (layer "F.Cu") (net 28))
 (segment (start 95.885685 48.26) (end 96.960106 49.334421) (width 0.2) (layer "F.Cu") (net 28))
 (segment (start 70.166651 49.213349) (end 71.12 48.26) (width 0.2) (layer "F.Cu") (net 28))
 (segment (start 71.12 48.26) (end 95.885685 48.26) (width 0.2) (layer "F.Cu") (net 28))
 (segment (start 70.166651 51.753349) (end 70.166651 49.213349) (width 0.2) (layer "F.Cu") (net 28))
 (segment (start 64.633417 55.788045) (end 66.131955 55.788045) (width 0.2) (layer "F.Cu") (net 28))
 (segment (start 96.960106 72.641875) (end 99.009054 74.690823) (width 0.2) (layer "F.Cu") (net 28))
 (segment (start 66.131955 55.788045) (end 70.166651 51.753349) (width 0.2) (layer "F.Cu") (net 28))
 (segment (start 101.6 91.44) (end 101.560425 91.479575) (width 0.2) (layer "F.Cu") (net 17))
 (segment (start 64.633417 58.328045) (end 67.334036 58.328045) (width 0.2) (layer "F.Cu") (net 17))
 (segment (start 94.38 49.06) (end 96.12 50.8) (width 0.2) (layer "F.Cu") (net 17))
 (segment (start 71.12 54.542081) (end 71.12 50.8) (width 0.2) (layer "F.Cu") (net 17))
 (segment (start 96.12 50.8) (end 96.12 85.96) (width 0.2) (layer "F.Cu") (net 17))
 (segment (start 96.12 85.96) (end 101.6 91.44) (width 0.2) (layer "F.Cu") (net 17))
 (segment (start 67.334036 58.328045) (end 71.12 54.542081) (width 0.2) (layer "F.Cu") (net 17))
 (segment (start 101.560425 91.479575) (end 101.560425 92.499983) (width 0.2) (layer "F.Cu") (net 17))
 (segment (start 72.86 49.06) (end 94.38 49.06) (width 0.2) (layer "F.Cu") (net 17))
 (segment (start 71.12 50.8) (end 72.86 49.06) (width 0.2) (layer "F.Cu") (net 17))
 (segment (start 86.139427 111.539427) (end 83.82 109.22) (width 0.2) (layer "F.Cu") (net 3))
 (segment (start 83.775455 93.935455) (end 79.873417 93.935455) (width 0.2) (layer "F.Cu") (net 3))
 (segment (start 87.416 111.539427) (end 86.139427 111.539427) (width 0.2) (layer "F.Cu") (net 3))
 (segment (start 83.82 109.22) (end 83.82 93.98) (width 0.2) (layer "F.Cu") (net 3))
 (segment (start 83.82 93.98) (end 83.775455 93.935455) (width 0.2) (layer "F.Cu") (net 3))
 (segment (start 79.965372 91.48741) (end 84.799852 91.48741) (width 0.2) (layer "F.Cu") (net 1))
 (segment (start 79.873417 91.395455) (end 79.965372 91.48741) (width 0.2) (layer "F.Cu") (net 1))
 (segment (start 84.799852 91.48741) (end 85.812425 92.499983) (width 0.2) (layer "F.Cu") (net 1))
 (segment (start 63.145915 71.028045) (end 58.42 75.75396) (width 0.2) (layer "F.Cu") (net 22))
 (segment (start 64.633417 71.028045) (end 63.145915 71.028045) (width 0.2) (layer "F.Cu") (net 22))
 (segment (start 55.88 83.82) (end 55.88 106.68) (width 0.2) (layer "F.Cu") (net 22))
 (segment (start 58.42 81.28) (end 55.88 83.82) (width 0.2) (layer "F.Cu") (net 22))
 (segment (start 55.88 106.68) (end 71.12 121.92) (width 0.2) (layer "F.Cu") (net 22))
 (segment (start 58.42 75.75396) (end 58.42 81.28) (width 0.2) (layer "F.Cu") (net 22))
 (segment (start 64.541462 78.74) (end 64.633417 78.648045) (width 0.2) (layer "F.Cu") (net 29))
 (segment (start 64.633417 76.108045) (end 61.563737 79.177725) (width 0.2) (layer "F.Cu") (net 27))
 (segment (start 58.82 102) (end 73.66 116.84) (width 0.2) (layer "F.Cu") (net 27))
 (segment (start 61.563737 83.674141) (end 61.617641 83.728045) (width 0.2) (layer "F.Cu") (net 27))
 (segment (start 58.82 86.525686) (end 58.82 102) (width 0.2) (layer "F.Cu") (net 27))
 (segment (start 61.563737 79.177725) (end 61.563737 83.674141) (width 0.2) (layer "F.Cu") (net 27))
 (segment (start 73.66 116.84) (end 73.66 127) (width 0.2) (layer "F.Cu") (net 27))
 (segment (start 61.617641 83.728045) (end 58.82 86.525686) (width 0.2) (layer "F.Cu") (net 27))
 (segment (start 73.66 127) (end 78.74 127) (width 0.2) (layer "F.Cu") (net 27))
 (segment (start 98.609054 48.14526) (end 98.609054 64.130823) (width 0.2) (layer "F.Cu") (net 18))
 (segment (start 98.389246 47.589246) (end 98.777157 47.977157) (width 0.2) (layer "F.Cu") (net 18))
 (segment (start 69.29876 50.08124) (end 69.29876 47.589246) (width 0.2) (layer "F.Cu") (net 18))
 (segment (start 69.29876 47.589246) (end 98.389246 47.589246) (width 0.2) (layer "F.Cu") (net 18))
 (segment (start 66.131955 53.248045) (end 69.29876 50.08124) (width 0.2) (layer "F.Cu") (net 18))
 (segment (start 64.633417 53.248045) (end 66.131955 53.248045) (width 0.2) (layer "F.Cu") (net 18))
 (segment (start 98.609054 64.130823) (end 99.009054 64.530823) (width 0.2) (layer "F.Cu") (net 18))
 (segment (start 98.777157 47.977157) (end 98.609054 48.14526) (width 0.2) (layer "F.Cu") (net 18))
 (segment (start 104.18 106.72) (end 104.18 111.539427) (width 0.2) (layer "F.Cu") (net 19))
 (segment (start 66.131955 60.868045) (end 72.197679 54.802321) (width 0.2) (layer "F.Cu") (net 19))
 (segment (start 94.972454 51.226769) (end 94.972454 92.432454) (width 0.2) (layer "F.Cu") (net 19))
 (segment (start 93.494329 49.748644) (end 94.972454 51.226769) (width 0.2) (layer "F.Cu") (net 19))
 (segment (start 94.972454 92.432454) (end 104.14 101.6) (width 0.2) (layer "F.Cu") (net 19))
 (segment (start 104.14 106.68) (end 104.18 106.72) (width 0.2) (layer "F.Cu") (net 19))
 (segment (start 104.14 101.6) (end 104.14 106.68) (width 0.2) (layer "F.Cu") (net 19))
 (segment (start 74.145671 49.748644) (end 93.494329 49.748644) (width 0.2) (layer "F.Cu") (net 19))
 (segment (start 72.197679 54.802321) (end 72.197679 51.696636) (width 0.2) (layer "F.Cu") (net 19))
 (segment (start 64.633417 60.868045) (end 66.131955 60.868045) (width 0.2) (layer "F.Cu") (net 19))
 (segment (start 72.197679 51.696636) (end 74.145671 49.748644) (width 0.2) (layer "F.Cu") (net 19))
 (segment (start 64.633417 73.568045) (end 64.541462 73.66) (width 0.2) (layer "F.Cu") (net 21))
 (segment (start 64.540279 73.661183) (end 64.633417 73.568045) (width 0.2) (layer "F.Cu") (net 21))
 (segment (start 57.326691 85.34419) (end 57.446346 85.463845) (width 0.2) (layer "F.Cu") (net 21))
 (segment (start 59.956323 82.714558) (end 57.326691 85.34419) (width 0.2) (layer "F.Cu") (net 21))
 (segment (start 57.446346 105.706346) (end 71.12 119.38) (width 0.2) (layer "F.Cu") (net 21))
 (segment (start 59.956323 77.274632) (end 59.956323 82.714558) (width 0.2) (layer "F.Cu") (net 21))
 (segment (start 63.5 73.66) (end 60.96 76.2) (width 0.2) (layer "F.Cu") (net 21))
 (segment (start 60.96 76.2) (end 60.96 76.270955) (width 0.2) (layer "F.Cu") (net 21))
 (segment (start 60.96 76.270955) (end 59.956323 77.274632) (width 0.2) (layer "F.Cu") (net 21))
 (segment (start 64.541462 73.66) (end 63.5 73.66) (width 0.2) (layer "F.Cu") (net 21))
 (segment (start 57.446346 85.463845) (end 57.446346 105.706346) (width 0.2) (layer "F.Cu") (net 21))
 (segment (start 78.74 66.04) (end 71.12 73.66) (width 0.2) (layer "F.Cu") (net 11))
 (segment (start 71.12 101.034314) (end 83.82 113.734314) (width 0.2) (layer "F.Cu") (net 11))
 (segment (start 83.82 113.734314) (end 83.82 124.46) (width 0.2) (layer "F.Cu") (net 11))
 (segment (start 79.828872 66.04) (end 78.74 66.04) (width 0.2) (layer "F.Cu") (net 11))
 (segment (start 79.873417 65.995455) (end 79.828872 66.04) (width 0.2) (layer "F.Cu") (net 11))
 (segment (start 83.82 124.46) (end 85.52305 124.46) (width 0.2) (layer "F.Cu") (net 11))
 (segment (start 71.12 73.66) (end 71.12 101.034314) (width 0.2) (layer "F.Cu") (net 11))
 (segment (start 79.917962 53.34) (end 79.873417 53.295455) (width 0.2) (layer "F.Cu") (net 16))
 (segment (start 83.82 53.34) (end 79.917962 53.34) (width 0.2) (layer "F.Cu") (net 16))
 (segment (start 84.277054 64.530823) (end 84.277054 53.797054) (width 0.2) (layer "F.Cu") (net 16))
 (segment (start 84.277054 53.797054) (end 83.82 53.34) (width 0.2) (layer "F.Cu") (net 16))
 (segment (start 93.98 127) (end 90.991471 124.011471) (width 0.2) (layer "F.Cu") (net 10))
 (segment (start 73.66 73.66) (end 78.74 68.58) (width 0.2) (layer "F.Cu") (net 10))
 (segment (start 78.74 68.58) (end 79.828872 68.58) (width 0.2) (layer "F.Cu") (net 10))
 (segment (start 90.991471 119.569891) (end 73.66 102.23842) (width 0.2) (layer "F.Cu") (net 10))
 (segment (start 95.391417 130.438924) (end 93.98 129.027507) (width 0.2) (layer "F.Cu") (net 10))
 (segment (start 79.828872 68.58) (end 79.873417 68.535455) (width 0.2) (layer "F.Cu") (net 10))
 (segment (start 90.991471 124.011471) (end 90.991471 119.569891) (width 0.2) (layer "F.Cu") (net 10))
 (segment (start 73.66 102.23842) (end 73.66 73.66) (width 0.2) (layer "F.Cu") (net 10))
 (segment (start 93.98 129.027507) (end 93.98 127) (width 0.2) (layer "F.Cu") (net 10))
 (segment (start 79.873417 73.615455) (end 83.201686 73.615455) (width 0.2) (layer "F.Cu") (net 8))
 (segment (start 83.201686 73.615455) (end 84.277054 74.690823) (width 0.2) (layer "F.Cu") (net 8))
 (segment (start 84.277054 74.690823) (end 84.277054 74.117054) (width 0.2) (layer "F.Cu") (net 8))
 (segment (start 90.17 117.261471) (end 92.427156 117.261471) (width 0.2) (layer "F.Cu") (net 9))
 (segment (start 78.74 105.831471) (end 90.17 117.261471) (width 0.2) (layer "F.Cu") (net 9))
 (segment (start 92.925328 117.759643) (end 92.925328 123.646161) (width 0.2) (layer "F.Cu") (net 9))
 (segment (start 76.2 99.06) (end 78.74 101.6) (width 0.2) (layer "F.Cu") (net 9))
 (segment (start 78.74 71.16741) (end 76.2 73.70741) (width 0.2) (layer "F.Cu") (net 9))
 (segment (start 92.925328 123.646161) (end 97.931417 128.65225) (width 0.2) (layer "F.Cu") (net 9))
 (segment (start 97.931417 128.65225) (end 97.931417 130.438924) (width 0.2) (layer "F.Cu") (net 9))
 (segment (start 76.2 73.70741) (end 76.2 99.06) (width 0.2) (layer "F.Cu") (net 9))
 (segment (start 78.69259 71.16741) (end 78.74 71.16741) (width 0.2) (layer "F.Cu") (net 9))
 (segment (start 78.74 71.16741) (end 79.781462 71.16741) (width 0.2) (layer "F.Cu") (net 9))
 (segment (start 78.74 101.6) (end 78.74 105.831471) (width 0.2) (layer "F.Cu") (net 9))
 (segment (start 92.427156 117.261471) (end 92.925328 117.759643) (width 0.2) (layer "F.Cu") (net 9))
 (segment (start 79.781462 71.16741) (end 79.873417 71.075455) (width 0.2) (layer "F.Cu") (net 9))
 (segment (start 64.541462 86.36) (end 64.633417 86.268045) (width 0.2) (layer "F.Cu") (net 30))
 (segment (start 74.639396 115.279396) (end 60.96 101.6) (width 0.2) (layer "F.Cu") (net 26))
 (segment (start 60.96 88.9) (end 61.051955 88.808045) (width 0.2) (layer "F.Cu") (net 26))
 (segment (start 61.051955 88.808045) (end 64.633417 88.808045) (width 0.2) (layer "F.Cu") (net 26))
 (segment (start 60.96 101.6) (end 60.96 88.9) (width 0.2) (layer "F.Cu") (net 26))
 (segment (start 74.639396 124.144569) (end 74.639396 115.279396) (width 0.2) (layer "F.Cu") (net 26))
 (segment (start 78.74 124.46) (end 74.954827 124.46) (width 0.2) (layer "F.Cu") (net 26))
 (segment (start 64.541462 88.9) (end 64.633417 88.808045) (width 0.2) (layer "F.Cu") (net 26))
 (segment (start 74.954827 124.46) (end 74.639396 124.144569) (width 0.2) (layer "F.Cu") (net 26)))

